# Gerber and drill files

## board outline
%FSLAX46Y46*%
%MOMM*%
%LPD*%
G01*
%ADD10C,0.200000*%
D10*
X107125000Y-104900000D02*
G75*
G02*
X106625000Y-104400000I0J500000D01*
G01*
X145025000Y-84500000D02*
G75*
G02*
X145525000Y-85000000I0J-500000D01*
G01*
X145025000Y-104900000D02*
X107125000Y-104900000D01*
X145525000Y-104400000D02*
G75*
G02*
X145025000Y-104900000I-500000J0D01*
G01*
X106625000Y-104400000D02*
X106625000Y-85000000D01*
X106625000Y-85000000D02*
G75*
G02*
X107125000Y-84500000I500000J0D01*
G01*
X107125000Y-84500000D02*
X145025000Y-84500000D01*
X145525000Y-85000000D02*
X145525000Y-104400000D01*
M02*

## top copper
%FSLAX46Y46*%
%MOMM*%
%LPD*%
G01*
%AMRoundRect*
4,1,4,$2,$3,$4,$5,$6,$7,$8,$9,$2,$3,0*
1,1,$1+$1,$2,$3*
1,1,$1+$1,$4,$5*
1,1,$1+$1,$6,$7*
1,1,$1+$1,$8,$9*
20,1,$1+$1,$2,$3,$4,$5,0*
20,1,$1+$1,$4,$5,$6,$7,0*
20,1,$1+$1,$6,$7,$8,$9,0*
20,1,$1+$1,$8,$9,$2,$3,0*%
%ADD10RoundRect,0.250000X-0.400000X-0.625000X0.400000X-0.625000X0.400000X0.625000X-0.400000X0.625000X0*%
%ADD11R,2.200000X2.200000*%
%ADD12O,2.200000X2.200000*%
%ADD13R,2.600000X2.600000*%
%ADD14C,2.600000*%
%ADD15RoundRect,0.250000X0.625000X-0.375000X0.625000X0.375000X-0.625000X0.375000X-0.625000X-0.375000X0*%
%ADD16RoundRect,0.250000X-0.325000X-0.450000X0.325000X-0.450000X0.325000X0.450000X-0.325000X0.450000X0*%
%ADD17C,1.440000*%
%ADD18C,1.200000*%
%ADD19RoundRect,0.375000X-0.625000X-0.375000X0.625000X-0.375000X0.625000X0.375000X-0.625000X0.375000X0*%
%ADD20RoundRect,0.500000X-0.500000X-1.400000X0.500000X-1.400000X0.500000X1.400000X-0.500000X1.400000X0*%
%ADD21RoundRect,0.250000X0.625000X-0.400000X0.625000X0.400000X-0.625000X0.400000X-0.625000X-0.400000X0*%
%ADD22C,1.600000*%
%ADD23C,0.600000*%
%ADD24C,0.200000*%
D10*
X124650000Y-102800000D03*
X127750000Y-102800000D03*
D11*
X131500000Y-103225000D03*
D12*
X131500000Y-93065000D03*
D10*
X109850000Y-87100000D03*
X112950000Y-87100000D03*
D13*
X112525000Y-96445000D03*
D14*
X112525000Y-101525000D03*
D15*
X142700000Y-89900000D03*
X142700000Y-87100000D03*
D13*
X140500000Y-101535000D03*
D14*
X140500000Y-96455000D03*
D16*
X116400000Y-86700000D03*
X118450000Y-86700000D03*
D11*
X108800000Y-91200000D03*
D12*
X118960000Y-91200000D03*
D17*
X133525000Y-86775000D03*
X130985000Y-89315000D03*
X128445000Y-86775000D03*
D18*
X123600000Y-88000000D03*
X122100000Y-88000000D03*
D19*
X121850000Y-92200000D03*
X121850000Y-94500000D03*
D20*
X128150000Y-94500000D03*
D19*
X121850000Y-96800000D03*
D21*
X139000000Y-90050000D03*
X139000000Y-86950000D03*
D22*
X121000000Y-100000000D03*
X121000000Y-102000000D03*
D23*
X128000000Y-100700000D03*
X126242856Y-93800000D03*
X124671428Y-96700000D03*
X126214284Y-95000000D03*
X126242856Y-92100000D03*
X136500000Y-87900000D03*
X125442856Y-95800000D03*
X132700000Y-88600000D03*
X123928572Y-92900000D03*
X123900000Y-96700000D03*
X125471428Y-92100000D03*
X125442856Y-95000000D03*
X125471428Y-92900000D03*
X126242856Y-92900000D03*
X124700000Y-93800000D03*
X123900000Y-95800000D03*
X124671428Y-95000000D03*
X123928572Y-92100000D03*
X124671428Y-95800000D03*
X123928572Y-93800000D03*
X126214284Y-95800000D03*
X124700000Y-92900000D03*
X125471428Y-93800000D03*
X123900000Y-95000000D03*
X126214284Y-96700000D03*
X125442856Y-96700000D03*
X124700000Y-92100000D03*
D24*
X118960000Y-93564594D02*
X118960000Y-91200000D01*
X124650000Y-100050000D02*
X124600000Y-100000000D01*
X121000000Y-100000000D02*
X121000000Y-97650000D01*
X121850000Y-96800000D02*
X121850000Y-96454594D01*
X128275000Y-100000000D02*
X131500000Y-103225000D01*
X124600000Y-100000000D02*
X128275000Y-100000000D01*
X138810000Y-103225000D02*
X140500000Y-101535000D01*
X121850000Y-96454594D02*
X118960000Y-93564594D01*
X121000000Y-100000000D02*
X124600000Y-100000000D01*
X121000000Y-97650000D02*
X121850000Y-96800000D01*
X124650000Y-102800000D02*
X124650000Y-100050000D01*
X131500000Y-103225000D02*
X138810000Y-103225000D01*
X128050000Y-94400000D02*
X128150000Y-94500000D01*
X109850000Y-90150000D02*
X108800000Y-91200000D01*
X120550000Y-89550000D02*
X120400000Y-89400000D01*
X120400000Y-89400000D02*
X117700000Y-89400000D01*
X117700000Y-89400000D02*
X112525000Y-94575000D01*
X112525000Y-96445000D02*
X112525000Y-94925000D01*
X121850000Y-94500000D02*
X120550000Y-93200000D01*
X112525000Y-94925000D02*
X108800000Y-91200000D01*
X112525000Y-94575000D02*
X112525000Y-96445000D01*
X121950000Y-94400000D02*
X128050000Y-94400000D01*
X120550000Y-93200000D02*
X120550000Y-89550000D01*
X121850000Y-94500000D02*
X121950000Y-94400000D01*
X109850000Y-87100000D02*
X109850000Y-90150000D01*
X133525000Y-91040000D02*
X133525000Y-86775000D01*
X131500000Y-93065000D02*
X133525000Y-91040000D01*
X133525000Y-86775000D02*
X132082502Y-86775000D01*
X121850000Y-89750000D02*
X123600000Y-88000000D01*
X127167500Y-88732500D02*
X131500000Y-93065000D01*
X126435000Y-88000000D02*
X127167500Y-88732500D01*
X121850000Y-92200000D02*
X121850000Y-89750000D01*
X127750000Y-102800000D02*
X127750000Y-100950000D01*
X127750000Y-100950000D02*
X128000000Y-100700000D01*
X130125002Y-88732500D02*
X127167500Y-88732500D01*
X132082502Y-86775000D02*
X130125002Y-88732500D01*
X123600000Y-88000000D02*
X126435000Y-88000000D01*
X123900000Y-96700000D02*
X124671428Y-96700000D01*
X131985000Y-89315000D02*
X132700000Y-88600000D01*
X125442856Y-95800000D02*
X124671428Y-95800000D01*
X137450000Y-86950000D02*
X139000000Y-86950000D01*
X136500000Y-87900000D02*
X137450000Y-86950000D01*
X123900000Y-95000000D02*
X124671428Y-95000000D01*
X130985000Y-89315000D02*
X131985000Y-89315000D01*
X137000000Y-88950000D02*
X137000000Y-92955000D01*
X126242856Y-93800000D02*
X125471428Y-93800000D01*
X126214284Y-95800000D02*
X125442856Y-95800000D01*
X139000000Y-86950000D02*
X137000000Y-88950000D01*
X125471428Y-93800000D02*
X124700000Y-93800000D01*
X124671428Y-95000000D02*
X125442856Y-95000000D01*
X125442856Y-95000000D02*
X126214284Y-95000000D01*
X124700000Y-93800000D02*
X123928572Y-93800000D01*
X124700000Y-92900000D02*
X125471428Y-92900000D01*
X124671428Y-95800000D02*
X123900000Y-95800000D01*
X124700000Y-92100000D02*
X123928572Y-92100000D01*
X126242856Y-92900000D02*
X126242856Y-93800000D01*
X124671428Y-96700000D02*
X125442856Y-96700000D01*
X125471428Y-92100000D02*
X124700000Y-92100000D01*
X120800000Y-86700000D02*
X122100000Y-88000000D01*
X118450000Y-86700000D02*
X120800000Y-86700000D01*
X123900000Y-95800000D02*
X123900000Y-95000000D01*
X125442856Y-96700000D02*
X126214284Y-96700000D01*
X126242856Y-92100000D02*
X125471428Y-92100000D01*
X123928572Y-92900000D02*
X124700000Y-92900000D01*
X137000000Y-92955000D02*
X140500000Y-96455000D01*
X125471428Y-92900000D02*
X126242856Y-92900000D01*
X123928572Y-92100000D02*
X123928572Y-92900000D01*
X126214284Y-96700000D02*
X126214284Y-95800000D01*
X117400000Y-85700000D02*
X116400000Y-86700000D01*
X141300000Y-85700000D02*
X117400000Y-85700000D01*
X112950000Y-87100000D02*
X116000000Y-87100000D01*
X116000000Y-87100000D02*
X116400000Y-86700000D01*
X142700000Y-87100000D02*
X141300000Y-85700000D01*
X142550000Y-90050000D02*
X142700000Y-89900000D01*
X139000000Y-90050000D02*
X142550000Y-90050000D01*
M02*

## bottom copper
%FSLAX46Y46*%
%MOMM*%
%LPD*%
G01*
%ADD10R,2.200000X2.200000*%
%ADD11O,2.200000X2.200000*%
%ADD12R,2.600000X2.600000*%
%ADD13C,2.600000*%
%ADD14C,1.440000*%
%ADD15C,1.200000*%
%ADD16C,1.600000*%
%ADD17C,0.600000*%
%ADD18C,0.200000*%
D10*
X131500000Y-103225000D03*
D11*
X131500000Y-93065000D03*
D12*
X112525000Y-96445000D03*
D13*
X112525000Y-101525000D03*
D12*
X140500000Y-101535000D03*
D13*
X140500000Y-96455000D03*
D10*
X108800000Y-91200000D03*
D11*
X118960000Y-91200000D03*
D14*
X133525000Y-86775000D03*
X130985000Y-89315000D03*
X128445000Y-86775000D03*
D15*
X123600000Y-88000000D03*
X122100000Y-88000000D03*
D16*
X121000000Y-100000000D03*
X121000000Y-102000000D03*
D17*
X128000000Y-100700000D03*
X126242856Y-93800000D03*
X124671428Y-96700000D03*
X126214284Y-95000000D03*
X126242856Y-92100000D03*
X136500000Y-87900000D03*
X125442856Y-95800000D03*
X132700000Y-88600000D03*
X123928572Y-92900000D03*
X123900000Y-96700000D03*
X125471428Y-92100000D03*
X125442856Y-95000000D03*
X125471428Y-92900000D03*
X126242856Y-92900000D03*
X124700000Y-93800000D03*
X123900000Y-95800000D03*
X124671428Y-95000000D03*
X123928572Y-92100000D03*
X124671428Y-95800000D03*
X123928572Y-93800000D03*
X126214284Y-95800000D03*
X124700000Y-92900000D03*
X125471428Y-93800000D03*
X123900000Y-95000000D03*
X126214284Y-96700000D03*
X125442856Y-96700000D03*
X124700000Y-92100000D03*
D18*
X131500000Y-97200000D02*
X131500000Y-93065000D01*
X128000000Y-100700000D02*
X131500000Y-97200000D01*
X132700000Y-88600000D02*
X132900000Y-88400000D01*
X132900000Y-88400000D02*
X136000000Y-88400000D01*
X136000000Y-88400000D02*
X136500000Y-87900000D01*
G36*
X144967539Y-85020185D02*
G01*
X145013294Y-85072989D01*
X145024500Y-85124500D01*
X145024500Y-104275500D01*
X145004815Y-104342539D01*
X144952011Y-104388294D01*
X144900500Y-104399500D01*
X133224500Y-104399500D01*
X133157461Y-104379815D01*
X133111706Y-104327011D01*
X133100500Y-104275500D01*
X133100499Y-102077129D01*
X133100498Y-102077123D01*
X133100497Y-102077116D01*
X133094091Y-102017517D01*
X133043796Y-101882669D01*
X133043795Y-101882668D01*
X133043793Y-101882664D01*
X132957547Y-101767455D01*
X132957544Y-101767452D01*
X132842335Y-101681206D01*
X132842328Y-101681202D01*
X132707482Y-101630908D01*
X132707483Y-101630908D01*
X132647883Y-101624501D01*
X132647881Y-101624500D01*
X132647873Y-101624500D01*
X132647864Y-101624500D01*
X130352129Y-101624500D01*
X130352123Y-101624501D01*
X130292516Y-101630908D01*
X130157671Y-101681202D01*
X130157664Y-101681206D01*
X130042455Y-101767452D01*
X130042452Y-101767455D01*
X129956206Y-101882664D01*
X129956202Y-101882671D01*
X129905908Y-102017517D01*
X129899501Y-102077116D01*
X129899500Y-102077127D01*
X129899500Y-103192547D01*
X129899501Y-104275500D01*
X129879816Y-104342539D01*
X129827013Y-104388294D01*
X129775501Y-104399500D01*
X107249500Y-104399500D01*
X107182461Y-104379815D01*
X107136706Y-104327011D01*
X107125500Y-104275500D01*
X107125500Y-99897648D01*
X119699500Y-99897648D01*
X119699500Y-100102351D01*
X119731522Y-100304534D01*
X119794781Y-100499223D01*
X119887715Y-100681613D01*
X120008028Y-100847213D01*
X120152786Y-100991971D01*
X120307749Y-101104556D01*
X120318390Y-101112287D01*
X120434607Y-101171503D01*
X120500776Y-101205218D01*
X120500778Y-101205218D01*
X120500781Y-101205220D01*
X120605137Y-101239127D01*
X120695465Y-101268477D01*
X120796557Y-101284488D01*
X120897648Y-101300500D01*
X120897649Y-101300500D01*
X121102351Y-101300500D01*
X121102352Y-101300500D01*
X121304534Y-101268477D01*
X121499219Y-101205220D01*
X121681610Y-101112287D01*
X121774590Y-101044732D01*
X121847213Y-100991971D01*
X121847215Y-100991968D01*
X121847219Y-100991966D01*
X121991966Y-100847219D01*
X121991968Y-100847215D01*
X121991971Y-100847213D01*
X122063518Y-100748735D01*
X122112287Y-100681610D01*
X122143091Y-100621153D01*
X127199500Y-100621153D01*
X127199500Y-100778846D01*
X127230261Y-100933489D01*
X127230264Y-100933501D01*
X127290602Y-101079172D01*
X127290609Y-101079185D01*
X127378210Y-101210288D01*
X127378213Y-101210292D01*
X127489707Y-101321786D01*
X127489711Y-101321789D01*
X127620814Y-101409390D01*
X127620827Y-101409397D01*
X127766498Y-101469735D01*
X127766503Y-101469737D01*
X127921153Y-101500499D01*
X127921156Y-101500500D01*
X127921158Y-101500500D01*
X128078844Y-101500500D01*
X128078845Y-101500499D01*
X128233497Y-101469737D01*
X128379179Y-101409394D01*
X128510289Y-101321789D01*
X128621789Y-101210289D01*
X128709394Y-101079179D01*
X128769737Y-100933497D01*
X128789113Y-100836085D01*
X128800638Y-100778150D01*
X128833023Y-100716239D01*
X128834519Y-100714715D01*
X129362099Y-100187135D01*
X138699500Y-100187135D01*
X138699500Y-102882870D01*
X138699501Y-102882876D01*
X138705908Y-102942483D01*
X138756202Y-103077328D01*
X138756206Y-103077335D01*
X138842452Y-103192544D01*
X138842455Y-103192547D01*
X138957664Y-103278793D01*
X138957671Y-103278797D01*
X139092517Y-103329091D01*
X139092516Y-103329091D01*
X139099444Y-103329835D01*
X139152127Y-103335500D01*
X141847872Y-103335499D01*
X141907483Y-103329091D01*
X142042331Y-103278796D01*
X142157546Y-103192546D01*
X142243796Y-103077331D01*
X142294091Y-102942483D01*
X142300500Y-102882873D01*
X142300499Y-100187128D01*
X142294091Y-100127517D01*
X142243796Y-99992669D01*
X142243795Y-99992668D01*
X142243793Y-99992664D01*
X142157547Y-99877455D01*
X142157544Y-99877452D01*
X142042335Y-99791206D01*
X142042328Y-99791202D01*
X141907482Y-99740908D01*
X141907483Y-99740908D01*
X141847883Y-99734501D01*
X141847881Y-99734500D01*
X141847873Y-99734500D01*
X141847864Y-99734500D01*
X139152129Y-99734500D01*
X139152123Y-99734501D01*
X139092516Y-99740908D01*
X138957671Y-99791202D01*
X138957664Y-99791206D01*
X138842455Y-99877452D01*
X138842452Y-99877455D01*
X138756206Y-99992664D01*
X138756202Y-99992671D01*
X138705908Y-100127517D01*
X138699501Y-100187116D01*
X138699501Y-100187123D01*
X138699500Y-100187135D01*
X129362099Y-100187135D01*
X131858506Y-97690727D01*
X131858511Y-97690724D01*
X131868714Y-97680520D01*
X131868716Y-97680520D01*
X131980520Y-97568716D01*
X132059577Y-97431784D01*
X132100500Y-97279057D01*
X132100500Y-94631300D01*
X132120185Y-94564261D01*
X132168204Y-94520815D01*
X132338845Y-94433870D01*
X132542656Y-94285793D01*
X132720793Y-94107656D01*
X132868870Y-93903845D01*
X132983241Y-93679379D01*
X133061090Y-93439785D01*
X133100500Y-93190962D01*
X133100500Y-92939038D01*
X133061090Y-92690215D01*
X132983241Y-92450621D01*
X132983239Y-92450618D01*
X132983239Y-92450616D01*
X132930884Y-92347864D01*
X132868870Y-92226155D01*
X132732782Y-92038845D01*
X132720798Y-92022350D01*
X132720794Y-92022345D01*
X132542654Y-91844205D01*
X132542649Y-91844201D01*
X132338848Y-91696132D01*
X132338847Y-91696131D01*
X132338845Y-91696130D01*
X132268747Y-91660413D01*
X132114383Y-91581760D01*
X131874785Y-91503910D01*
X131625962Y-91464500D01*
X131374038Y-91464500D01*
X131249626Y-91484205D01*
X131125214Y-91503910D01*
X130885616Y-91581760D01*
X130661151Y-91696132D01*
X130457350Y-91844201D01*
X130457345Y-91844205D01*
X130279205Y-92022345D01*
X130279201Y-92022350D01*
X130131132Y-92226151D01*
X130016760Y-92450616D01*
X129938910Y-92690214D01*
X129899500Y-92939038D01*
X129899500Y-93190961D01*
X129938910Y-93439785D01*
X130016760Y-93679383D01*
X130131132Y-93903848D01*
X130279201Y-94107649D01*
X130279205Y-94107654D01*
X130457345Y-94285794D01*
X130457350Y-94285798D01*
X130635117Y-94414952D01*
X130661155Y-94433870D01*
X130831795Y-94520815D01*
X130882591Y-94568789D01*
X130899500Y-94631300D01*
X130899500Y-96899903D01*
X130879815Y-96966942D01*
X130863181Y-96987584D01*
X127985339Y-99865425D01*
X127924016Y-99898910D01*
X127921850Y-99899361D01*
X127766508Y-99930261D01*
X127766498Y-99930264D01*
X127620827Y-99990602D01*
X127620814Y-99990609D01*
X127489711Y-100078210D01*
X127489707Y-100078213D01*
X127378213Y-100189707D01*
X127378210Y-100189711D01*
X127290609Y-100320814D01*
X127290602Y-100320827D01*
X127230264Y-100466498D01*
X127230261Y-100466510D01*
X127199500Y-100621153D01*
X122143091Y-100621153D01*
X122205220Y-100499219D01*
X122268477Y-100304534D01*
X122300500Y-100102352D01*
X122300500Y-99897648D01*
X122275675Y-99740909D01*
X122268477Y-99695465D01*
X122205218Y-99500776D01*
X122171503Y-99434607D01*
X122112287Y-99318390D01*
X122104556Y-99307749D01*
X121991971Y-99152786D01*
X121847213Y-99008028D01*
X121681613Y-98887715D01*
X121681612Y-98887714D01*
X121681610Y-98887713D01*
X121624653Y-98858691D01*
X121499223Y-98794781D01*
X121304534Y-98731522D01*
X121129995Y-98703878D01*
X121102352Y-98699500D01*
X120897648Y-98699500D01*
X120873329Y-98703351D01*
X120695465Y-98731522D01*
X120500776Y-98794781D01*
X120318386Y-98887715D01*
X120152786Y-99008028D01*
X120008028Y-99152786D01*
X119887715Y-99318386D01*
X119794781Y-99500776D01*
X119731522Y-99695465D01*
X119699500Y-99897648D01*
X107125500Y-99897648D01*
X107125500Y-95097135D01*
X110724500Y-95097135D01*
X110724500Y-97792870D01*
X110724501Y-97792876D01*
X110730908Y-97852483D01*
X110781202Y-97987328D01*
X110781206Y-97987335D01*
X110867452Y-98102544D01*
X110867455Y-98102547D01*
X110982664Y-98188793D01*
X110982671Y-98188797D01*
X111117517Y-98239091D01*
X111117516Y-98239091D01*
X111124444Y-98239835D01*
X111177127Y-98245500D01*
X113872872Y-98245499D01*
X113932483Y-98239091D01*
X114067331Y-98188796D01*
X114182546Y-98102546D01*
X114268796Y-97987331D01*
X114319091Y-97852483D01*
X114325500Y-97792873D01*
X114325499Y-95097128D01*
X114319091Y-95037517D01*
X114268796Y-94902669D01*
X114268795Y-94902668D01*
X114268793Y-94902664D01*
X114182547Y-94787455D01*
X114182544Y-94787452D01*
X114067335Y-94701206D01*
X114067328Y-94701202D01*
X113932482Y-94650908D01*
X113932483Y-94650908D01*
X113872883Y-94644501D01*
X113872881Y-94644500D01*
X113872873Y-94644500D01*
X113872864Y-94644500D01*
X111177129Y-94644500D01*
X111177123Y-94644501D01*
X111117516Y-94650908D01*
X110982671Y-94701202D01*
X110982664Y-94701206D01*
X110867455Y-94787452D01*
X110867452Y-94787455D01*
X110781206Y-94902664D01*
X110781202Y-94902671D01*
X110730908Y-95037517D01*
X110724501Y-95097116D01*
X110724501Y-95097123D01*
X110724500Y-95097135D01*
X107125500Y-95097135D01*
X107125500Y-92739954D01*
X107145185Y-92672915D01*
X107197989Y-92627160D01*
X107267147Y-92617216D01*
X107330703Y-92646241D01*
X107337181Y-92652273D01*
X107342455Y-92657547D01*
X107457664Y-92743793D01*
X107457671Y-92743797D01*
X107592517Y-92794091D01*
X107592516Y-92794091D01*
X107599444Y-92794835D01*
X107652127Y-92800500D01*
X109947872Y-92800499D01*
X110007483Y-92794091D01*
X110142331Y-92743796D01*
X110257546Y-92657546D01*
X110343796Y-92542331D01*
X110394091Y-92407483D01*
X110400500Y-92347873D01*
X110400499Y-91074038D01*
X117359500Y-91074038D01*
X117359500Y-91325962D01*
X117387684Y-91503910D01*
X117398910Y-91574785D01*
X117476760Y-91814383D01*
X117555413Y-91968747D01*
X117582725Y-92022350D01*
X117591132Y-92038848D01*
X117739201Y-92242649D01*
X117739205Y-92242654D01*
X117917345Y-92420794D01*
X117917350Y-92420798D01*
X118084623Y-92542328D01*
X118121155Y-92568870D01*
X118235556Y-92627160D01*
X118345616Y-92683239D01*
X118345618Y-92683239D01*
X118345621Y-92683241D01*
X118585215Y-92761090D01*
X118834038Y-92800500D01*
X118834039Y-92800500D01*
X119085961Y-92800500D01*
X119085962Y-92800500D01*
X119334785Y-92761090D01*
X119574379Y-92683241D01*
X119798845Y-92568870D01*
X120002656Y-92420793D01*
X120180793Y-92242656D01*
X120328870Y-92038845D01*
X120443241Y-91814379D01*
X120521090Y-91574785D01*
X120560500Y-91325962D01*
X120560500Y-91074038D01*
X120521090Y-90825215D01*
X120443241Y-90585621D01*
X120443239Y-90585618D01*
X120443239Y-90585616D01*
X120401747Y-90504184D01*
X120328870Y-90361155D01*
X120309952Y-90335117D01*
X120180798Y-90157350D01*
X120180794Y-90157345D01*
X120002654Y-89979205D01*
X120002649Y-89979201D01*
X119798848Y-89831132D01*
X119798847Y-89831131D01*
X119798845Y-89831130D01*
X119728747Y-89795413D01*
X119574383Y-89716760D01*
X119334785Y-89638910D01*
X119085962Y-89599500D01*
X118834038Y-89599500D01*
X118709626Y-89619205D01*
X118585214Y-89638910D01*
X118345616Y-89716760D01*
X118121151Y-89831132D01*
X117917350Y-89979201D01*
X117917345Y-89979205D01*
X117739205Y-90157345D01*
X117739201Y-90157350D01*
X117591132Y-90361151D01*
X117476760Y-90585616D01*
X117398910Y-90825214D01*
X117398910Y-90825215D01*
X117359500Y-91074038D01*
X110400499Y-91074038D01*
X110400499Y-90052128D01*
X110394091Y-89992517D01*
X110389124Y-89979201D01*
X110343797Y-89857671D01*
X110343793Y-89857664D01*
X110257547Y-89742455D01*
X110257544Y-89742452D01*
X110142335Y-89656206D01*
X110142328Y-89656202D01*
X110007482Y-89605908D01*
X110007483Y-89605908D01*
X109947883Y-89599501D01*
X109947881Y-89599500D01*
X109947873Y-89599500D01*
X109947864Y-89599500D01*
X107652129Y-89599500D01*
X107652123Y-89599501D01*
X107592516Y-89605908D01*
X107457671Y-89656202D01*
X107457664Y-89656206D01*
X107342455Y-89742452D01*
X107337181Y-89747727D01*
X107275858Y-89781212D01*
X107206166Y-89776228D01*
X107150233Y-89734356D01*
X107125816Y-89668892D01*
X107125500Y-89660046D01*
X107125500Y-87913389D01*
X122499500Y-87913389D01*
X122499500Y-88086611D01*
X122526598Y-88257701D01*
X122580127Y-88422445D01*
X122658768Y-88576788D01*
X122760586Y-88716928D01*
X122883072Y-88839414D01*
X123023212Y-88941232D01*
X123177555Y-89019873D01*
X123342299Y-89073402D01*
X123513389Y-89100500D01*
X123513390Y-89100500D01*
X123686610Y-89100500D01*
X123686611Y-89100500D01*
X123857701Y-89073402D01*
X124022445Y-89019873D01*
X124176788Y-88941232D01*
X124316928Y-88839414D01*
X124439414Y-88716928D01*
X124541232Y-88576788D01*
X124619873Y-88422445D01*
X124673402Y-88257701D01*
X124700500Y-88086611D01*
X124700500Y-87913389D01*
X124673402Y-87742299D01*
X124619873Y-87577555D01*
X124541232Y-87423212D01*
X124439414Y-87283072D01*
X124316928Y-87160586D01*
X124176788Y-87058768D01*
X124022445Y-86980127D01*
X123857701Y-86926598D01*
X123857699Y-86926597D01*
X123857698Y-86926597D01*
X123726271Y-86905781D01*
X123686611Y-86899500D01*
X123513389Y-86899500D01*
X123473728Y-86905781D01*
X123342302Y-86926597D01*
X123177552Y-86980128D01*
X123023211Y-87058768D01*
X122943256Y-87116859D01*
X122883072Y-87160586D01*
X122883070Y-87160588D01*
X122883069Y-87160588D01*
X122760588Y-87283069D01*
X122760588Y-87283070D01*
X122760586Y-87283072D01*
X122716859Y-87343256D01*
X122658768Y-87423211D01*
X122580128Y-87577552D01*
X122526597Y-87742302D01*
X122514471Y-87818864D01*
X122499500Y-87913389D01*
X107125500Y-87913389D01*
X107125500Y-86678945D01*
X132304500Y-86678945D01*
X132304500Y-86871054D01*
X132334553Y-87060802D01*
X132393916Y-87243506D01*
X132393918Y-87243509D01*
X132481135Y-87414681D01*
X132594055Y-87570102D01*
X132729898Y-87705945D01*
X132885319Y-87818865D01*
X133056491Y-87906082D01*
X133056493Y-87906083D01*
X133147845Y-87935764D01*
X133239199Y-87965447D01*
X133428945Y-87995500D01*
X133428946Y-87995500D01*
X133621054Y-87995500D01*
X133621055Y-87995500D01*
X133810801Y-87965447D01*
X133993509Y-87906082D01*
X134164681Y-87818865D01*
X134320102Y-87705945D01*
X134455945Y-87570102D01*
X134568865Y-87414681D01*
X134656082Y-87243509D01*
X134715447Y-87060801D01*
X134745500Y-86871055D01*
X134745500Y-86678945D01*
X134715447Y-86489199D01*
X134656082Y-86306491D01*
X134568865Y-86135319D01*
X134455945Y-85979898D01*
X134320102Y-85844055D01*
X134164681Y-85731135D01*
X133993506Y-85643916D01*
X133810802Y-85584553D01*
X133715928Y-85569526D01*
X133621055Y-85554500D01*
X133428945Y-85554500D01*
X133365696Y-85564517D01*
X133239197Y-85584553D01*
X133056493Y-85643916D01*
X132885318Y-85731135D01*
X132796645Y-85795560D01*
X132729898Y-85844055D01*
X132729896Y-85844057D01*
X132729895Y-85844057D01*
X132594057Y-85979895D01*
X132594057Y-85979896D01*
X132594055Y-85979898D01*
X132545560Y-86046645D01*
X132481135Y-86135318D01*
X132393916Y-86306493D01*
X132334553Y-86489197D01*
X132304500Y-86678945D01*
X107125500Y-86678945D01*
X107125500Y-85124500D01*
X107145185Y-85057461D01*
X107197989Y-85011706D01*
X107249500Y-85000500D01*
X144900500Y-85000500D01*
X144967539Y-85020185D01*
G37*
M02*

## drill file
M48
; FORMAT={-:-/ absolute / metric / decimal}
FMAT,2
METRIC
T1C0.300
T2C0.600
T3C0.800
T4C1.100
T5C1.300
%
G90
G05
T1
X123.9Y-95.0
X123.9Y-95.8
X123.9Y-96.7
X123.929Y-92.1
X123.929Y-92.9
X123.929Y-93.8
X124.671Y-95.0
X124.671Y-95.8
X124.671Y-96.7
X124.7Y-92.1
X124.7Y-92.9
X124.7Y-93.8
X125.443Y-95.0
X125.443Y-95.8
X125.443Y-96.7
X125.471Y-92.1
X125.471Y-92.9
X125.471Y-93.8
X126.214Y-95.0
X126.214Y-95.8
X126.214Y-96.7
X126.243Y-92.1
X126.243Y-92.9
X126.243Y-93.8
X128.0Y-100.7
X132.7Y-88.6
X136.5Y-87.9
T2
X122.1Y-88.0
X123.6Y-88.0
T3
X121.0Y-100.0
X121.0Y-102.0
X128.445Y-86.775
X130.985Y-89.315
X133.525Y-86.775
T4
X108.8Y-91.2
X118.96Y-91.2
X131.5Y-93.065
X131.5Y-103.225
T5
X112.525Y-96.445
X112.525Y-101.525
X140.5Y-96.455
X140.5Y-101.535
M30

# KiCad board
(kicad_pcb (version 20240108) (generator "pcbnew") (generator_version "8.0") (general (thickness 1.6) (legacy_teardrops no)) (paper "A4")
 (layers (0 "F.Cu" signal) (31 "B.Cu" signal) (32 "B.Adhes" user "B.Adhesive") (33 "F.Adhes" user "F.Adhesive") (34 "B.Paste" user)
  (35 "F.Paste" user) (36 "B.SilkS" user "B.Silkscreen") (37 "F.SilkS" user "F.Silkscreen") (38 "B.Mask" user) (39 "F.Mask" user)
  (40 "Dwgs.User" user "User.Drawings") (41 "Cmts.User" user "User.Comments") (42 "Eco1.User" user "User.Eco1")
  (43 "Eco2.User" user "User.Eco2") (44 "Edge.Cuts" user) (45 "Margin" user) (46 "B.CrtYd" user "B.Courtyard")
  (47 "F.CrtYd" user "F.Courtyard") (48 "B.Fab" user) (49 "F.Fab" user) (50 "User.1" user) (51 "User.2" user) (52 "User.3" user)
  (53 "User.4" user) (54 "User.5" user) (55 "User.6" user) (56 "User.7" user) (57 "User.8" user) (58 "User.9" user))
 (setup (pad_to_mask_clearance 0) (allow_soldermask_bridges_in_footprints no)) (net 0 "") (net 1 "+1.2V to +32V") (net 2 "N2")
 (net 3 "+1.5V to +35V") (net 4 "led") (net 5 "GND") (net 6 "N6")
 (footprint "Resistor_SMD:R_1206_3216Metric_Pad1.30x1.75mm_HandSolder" (layer "F.Cu") (at 126.2 102.8)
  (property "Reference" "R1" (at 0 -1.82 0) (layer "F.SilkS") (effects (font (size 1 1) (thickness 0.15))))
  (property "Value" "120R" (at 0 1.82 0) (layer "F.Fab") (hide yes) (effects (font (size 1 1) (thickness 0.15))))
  (pad "1" smd roundrect (at -1.55 0) (size 1.3 1.75) (layers "F.Cu" "F.Paste" "F.Mask") (roundrect_rratio 0.192308) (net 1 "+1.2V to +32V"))
  (pad "2" smd roundrect (at 1.55 0) (size 1.3 1.75) (layers "F.Cu" "F.Paste" "F.Mask") (roundrect_rratio 0.192308) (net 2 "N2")))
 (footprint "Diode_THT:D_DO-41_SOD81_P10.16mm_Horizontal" (layer "F.Cu") (at 131.5 103.225 90)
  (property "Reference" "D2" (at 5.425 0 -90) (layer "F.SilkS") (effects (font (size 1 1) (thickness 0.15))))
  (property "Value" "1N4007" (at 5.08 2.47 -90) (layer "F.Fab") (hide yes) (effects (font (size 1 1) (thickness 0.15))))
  (pad "1" thru_hole rect (at 0 0 90) (size 2.2 2.2) (drill 1.1) (layers "*.Cu" "*.Mask") (remove_unused_layers no) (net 1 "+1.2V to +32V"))
  (pad "2" thru_hole oval (at 10.16 0 90) (size 2.2 2.2) (drill 1.1) (layers "*.Cu" "*.Mask") (remove_unused_layers no) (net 2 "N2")))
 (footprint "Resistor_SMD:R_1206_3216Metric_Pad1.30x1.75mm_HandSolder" (layer "F.Cu") (at 111.4 87.1)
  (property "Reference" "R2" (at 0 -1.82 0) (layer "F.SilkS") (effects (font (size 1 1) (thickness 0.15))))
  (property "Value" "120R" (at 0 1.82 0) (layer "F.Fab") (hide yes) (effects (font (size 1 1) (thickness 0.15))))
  (pad "1" smd roundrect (at -1.55 0) (size 1.3 1.75) (layers "F.Cu" "F.Paste" "F.Mask") (roundrect_rratio 0.192308) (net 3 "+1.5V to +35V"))
  (pad "2" smd roundrect (at 1.55 0) (size 1.3 1.75) (layers "F.Cu" "F.Paste" "F.Mask") (roundrect_rratio 0.192308) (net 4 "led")))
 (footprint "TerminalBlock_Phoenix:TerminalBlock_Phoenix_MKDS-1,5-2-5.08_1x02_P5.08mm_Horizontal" (layer "F.Cu") (at 112.525 96.445 -90)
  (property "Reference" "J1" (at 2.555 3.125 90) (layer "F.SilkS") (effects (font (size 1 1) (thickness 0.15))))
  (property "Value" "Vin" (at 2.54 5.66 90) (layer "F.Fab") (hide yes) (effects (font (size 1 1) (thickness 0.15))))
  (pad "1" thru_hole rect (at 0 0 270) (size 2.6 2.6) (drill 1.3) (layers "*.Cu" "*.Mask") (remove_unused_layers no) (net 3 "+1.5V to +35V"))
  (pad "2" thru_hole circle (at 5.08 0 270) (size 2.6 2.6) (drill 1.3) (layers "*.Cu" "*.Mask") (remove_unused_layers no) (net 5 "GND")))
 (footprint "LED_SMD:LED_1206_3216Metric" (layer "F.Cu") (at 142.7 88.5 90)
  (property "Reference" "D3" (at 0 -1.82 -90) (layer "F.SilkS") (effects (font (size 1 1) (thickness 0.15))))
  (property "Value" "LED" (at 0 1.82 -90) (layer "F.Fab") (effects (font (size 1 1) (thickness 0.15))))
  (pad "1" smd roundrect (at -1.4 0 90) (size 1.25 1.75) (layers "F.Cu" "F.Paste" "F.Mask") (roundrect_rratio 0.2) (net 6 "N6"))
  (pad "2" smd roundrect (at 1.4 0 90) (size 1.25 1.75) (layers "F.Cu" "F.Paste" "F.Mask") (roundrect_rratio 0.2) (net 4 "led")))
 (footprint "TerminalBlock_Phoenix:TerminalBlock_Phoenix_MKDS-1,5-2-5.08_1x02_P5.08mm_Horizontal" (layer "F.Cu") (at 140.5 101.535 90)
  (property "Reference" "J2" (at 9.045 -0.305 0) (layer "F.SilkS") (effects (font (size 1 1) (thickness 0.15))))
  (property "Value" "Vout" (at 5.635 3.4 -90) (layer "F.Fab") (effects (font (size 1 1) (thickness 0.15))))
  (pad "1" thru_hole rect (at 0 0 90) (size 2.6 2.6) (drill 1.3) (layers "*.Cu" "*.Mask") (remove_unused_layers no) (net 1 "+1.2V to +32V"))
  (pad "2" thru_hole circle (at 5.08 0 90) (size 2.6 2.6) (drill 1.3) (layers "*.Cu" "*.Mask") (remove_unused_layers no) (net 5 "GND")))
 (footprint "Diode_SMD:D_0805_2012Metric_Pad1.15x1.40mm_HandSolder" (layer "F.Cu") (at 117.425 86.7)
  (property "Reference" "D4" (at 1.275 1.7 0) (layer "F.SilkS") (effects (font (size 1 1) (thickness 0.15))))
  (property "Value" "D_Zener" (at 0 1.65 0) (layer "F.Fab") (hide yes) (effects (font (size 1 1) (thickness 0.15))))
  (pad "1" smd roundrect (at -1.025 0) (size 1.15 1.4) (layers "F.Cu" "F.Paste" "F.Mask") (roundrect_rratio 0.217391) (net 4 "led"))
  (pad "2" smd roundrect (at 1.025 0) (size 1.15 1.4) (layers "F.Cu" "F.Paste" "F.Mask") (roundrect_rratio 0.217391) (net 5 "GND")))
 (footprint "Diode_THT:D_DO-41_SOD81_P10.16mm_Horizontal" (layer "F.Cu") (at 108.8 91.2)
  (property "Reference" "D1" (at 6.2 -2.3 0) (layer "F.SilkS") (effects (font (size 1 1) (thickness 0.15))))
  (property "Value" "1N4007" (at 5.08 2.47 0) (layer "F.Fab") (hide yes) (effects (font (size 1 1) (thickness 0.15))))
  (pad "1" thru_hole rect (at 0 0) (size 2.2 2.2) (drill 1.1) (layers "*.Cu" "*.Mask") (remove_unused_layers no) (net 3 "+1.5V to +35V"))
  (pad "2" thru_hole oval (at 10.16 0) (size 2.2 2.2) (drill 1.1) (layers "*.Cu" "*.Mask") (remove_unused_layers no) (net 1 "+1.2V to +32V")))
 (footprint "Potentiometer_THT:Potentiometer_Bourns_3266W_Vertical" (layer "F.Cu") (at 133.525 86.775)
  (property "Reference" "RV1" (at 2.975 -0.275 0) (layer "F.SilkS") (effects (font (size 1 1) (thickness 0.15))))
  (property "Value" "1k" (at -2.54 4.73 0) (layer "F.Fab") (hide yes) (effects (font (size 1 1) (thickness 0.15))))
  (pad "1" thru_hole circle (at 0 0) (size 1.44 1.44) (drill 0.8) (layers "*.Cu" "*.Mask") (remove_unused_layers no) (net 2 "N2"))
  (pad "2" thru_hole circle (at -2.54 2.54) (size 1.44 1.44) (drill 0.8) (layers "*.Cu" "*.Mask") (remove_unused_layers no) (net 5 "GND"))
  (pad "3" thru_hole circle (at -5.08 0) (size 1.44 1.44) (drill 0.8) (layers "*.Cu" "*.Mask") (remove_unused_layers no) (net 5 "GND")))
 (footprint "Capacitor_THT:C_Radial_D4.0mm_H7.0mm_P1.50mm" (layer "F.Cu") (at 123.6 88 180)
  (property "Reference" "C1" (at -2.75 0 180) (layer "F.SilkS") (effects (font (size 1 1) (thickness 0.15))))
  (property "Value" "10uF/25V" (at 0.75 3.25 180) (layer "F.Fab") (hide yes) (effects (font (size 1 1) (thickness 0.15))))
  (pad "1" thru_hole circle (at 0 0 180) (size 1.2 1.2) (drill 0.6) (layers "*.Cu" "*.Mask") (remove_unused_layers no) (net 2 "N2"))
  (pad "2" thru_hole circle (at 1.5 0 180) (size 1.2 1.2) (drill 0.6) (layers "*.Cu" "*.Mask") (remove_unused_layers no) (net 5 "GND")))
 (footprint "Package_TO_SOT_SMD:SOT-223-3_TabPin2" (layer "F.Cu") (at 125 94.5)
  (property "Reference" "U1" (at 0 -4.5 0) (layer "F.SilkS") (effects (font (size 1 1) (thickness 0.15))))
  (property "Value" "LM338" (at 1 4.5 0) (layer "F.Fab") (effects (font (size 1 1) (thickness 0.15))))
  (pad "1" smd roundrect (at -3.15 -2.3) (size 2 1.5) (layers "F.Cu" "F.Paste" "F.Mask") (roundrect_rratio 0.25) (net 2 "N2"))
  (pad "2" smd roundrect (at -3.15 0) (size 2 1.5) (layers "F.Cu" "F.Paste" "F.Mask") (roundrect_rratio 0.25) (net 3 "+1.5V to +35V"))
  (pad "2" smd roundrect (at 3.15 0) (size 2 3.8) (layers "F.Cu" "F.Paste" "F.Mask") (roundrect_rratio 0.25) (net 3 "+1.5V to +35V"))
  (pad "3" smd roundrect (at -3.15 2.3) (size 2 1.5) (layers "F.Cu" "F.Paste" "F.Mask") (roundrect_rratio 0.25) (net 1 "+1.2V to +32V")))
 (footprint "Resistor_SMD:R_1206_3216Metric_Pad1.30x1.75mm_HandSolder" (layer "F.Cu") (at 139 88.5 90)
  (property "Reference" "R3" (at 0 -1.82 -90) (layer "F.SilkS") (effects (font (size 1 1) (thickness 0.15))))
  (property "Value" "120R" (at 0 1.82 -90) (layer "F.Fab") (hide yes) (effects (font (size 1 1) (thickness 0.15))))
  (pad "1" smd roundrect (at -1.55 0 90) (size 1.3 1.75) (layers "F.Cu" "F.Paste" "F.Mask") (roundrect_rratio 0.192308) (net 6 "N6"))
  (pad "2" smd roundrect (at 1.55 0 90) (size 1.3 1.75) (layers "F.Cu" "F.Paste" "F.Mask") (roundrect_rratio 0.192308) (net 5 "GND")))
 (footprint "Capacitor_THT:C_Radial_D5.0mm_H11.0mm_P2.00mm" (layer "F.Cu") (at 121 100 -90)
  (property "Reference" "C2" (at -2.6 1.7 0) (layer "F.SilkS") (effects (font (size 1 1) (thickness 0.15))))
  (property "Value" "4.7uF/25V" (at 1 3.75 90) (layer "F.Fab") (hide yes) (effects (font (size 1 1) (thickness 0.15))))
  (pad "1" thru_hole circle (at 0 0 270) (size 1.6 1.6) (drill 0.8) (layers "*.Cu" "*.Mask") (remove_unused_layers no)
   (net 1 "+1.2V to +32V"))
  (pad "2" thru_hole circle (at 2 0 270) (size 1.6 1.6) (drill 0.8) (layers "*.Cu" "*.Mask") (remove_unused_layers no) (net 5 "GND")))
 (gr_arc (start 107.125 104.9) (mid 106.771447 104.753553) (end 106.625 104.4) (stroke (width 0.2) (type default)) (layer "Edge.Cuts"))
 (gr_arc (start 145.025 84.5) (mid 145.378553 84.646447) (end 145.525 85) (stroke (width 0.2) (type default)) (layer "Edge.Cuts"))
 (gr_line (start 145.025 104.9) (end 107.125 104.9) (stroke (width 0.2) (type default)) (layer "Edge.Cuts"))
 (gr_arc (start 145.525 104.4) (mid 145.378553 104.753553) (end 145.025 104.9) (stroke (width 0.2) (type default)) (layer "Edge.Cuts"))
 (gr_line (start 106.625 104.4) (end 106.625 85) (stroke (width 0.2) (type default)) (layer "Edge.Cuts"))
 (gr_arc (start 106.625 85) (mid 106.771447 84.646447) (end 107.125 84.5) (stroke (width 0.2) (type default)) (layer "Edge.Cuts"))
 (gr_line (start 107.125 84.5) (end 145.025 84.5) (stroke (width 0.2) (type default)) (layer "Edge.Cuts"))
 (gr_line (start 145.525 85) (end 145.525 104.4) (stroke (width 0.2) (type default)) (layer "Edge.Cuts"))
 (segment (start 118.96 93.564594) (end 118.96 91.2) (width 0.2) (layer "F.Cu") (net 1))
 (segment (start 124.65 100.05) (end 124.6 100) (width 0.2) (layer "F.Cu") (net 1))
 (segment (start 121 100) (end 121 97.65) (width 0.2) (layer "F.Cu") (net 1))
 (segment (start 121.85 96.8) (end 121.85 96.454594) (width 0.2) (layer "F.Cu") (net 1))
 (segment (start 128.275 100) (end 131.5 103.225) (width 0.2) (layer "F.Cu") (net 1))
 (segment (start 124.6 100) (end 128.275 100) (width 0.2) (layer "F.Cu") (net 1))
 (segment (start 138.81 103.225) (end 140.5 101.535) (width 0.2) (layer "F.Cu") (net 1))
 (segment (start 121.85 96.454594) (end 118.96 93.564594) (width 0.2) (layer "F.Cu") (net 1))
 (segment (start 121 100) (end 124.6 100) (width 0.2) (layer "F.Cu") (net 1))
 (segment (start 121 97.65) (end 121.85 96.8) (width 0.2) (layer "F.Cu") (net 1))
 (segment (start 124.65 102.8) (end 124.65 100.05) (width 0.2) (layer "F.Cu") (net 1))
 (segment (start 131.5 103.225) (end 138.81 103.225) (width 0.2) (layer "F.Cu") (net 1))
 (segment (start 128.05 94.4) (end 128.15 94.5) (width 0.2) (layer "F.Cu") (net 3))
 (segment (start 109.85 90.15) (end 108.8 91.2) (width 0.2) (layer "F.Cu") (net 3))
 (segment (start 120.55 89.55) (end 120.4 89.4) (width 0.2) (layer "F.Cu") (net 3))
 (segment (start 120.4 89.4) (end 117.7 89.4) (width 0.2) (layer "F.Cu") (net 3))
 (segment (start 117.7 89.4) (end 112.525 94.575) (width 0.2) (layer "F.Cu") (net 3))
 (segment (start 112.525 96.445) (end 112.525 94.925) (width 0.2) (layer "F.Cu") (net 3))
 (segment (start 121.85 94.5) (end 120.55 93.2) (width 0.2) (layer "F.Cu") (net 3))
 (segment (start 112.525 94.925) (end 108.8 91.2) (width 0.2) (layer "F.Cu") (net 3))
 (segment (start 112.525 94.575) (end 112.525 96.445) (width 0.2) (layer "F.Cu") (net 3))
 (segment (start 121.95 94.4) (end 128.05 94.4) (width 0.2) (layer "F.Cu") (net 3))
 (segment (start 120.55 93.2) (end 120.55 89.55) (width 0.2) (layer "F.Cu") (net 3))
 (segment (start 121.85 94.5) (end 121.95 94.4) (width 0.2) (layer "F.Cu") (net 3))
 (segment (start 109.85 87.1) (end 109.85 90.15) (width 0.2) (layer "F.Cu") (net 3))
 (segment (start 133.525 91.04) (end 133.525 86.775) (width 0.2) (layer "F.Cu") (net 2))
 (segment (start 131.5 93.065) (end 133.525 91.04) (width 0.2) (layer "F.Cu") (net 2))
 (segment (start 133.525 86.775) (end 132.082502 86.775) (width 0.2) (layer "F.Cu") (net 2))
 (segment (start 121.85 89.75) (end 123.6 88) (width 0.2) (layer "F.Cu") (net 2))
 (segment (start 127.1675 88.7325) (end 131.5 93.065) (width 0.2) (layer "F.Cu") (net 2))
 (segment (start 126.435 88) (end 127.1675 88.7325) (width 0.2) (layer "F.Cu") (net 2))
 (segment (start 121.85 92.2) (end 121.85 89.75) (width 0.2) (layer "F.Cu") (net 2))
 (segment (start 127.75 102.8) (end 127.75 100.95) (width 0.2) (layer "F.Cu") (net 2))
 (segment (start 127.75 100.95) (end 128 100.7) (width 0.2) (layer "F.Cu") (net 2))
 (segment (start 130.125002 88.7325) (end 127.1675 88.7325) (width 0.2) (layer "F.Cu") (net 2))
 (segment (start 132.082502 86.775) (end 130.125002 88.7325) (width 0.2) (layer "F.Cu") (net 2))
 (segment (start 123.6 88) (end 126.435 88) (width 0.2) (layer "F.Cu") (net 2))
 (via (at 128 100.7) (size 0.6) (drill 0.3) (layers "F.Cu" "B.Cu") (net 2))
 (segment (start 131.5 97.2) (end 131.5 93.065) (width 0.2) (layer "B.Cu") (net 2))
 (segment (start 128 100.7) (end 131.5 97.2) (width 0.2) (layer "B.Cu") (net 2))
 (segment (start 123.9 96.7) (end 124.671428 96.7) (width 0.2) (layer "F.Cu") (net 5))
 (segment (start 131.985 89.315) (end 132.7 88.6) (width 0.2) (layer "F.Cu") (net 5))
 (segment (start 125.442856 95.8) (end 124.671428 95.8) (width 0.2) (layer "F.Cu") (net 5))
 (segment (start 137.45 86.95) (end 139 86.95) (width 0.2) (layer "F.Cu") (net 5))
 (segment (start 136.5 87.9) (end 137.45 86.95) (width 0.2) (layer "F.Cu") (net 5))
 (segment (start 123.9 95) (end 124.671428 95) (width 0.2) (layer "F.Cu") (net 5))
 (segment (start 130.985 89.315) (end 131.985 89.315) (width 0.2) (layer "F.Cu") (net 5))
 (segment (start 137 88.95) (end 137 92.955) (width 0.2) (layer "F.Cu") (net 5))
 (segment (start 126.242856 93.8) (end 125.471428 93.8) (width 0.2) (layer "F.Cu") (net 5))
 (segment (start 126.214284 95.8) (end 125.442856 95.8) (width 0.2) (layer "F.Cu") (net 5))
 (segment (start 139 86.95) (end 137 88.95) (width 0.2) (layer "F.Cu") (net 5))
 (segment (start 125.471428 93.8) (end 124.7 93.8) (width 0.2) (layer "F.Cu") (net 5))
 (segment (start 124.671428 95) (end 125.442856 95) (width 0.2) (layer "F.Cu") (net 5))
 (segment (start 125.442856 95) (end 126.214284 95) (width 0.2) (layer "F.Cu") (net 5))
 (segment (start 124.7 93.8) (end 123.928572 93.8) (width 0.2) (layer "F.Cu") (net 5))
 (segment (start 124.7 92.9) (end 125.471428 92.9) (width 0.2) (layer "F.Cu") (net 5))
 (segment (start 124.671428 95.8) (end 123.9 95.8) (width 0.2) (layer "F.Cu") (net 5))
 (segment (start 124.7 92.1) (end 123.928572 92.1) (width 0.2) (layer "F.Cu") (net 5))
 (segment (start 126.242856 92.9) (end 126.242856 93.8) (width 0.2) (layer "F.Cu") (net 5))
 (segment (start 124.671428 96.7) (end 125.442856 96.7) (width 0.2) (layer "F.Cu") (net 5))
 (segment (start 125.471428 92.1) (end 124.7 92.1) (width 0.2) (layer "F.Cu") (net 5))
 (segment (start 120.8 86.7) (end 122.1 88) (width 0.2) (layer "F.Cu") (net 5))
 (segment (start 118.45 86.7) (end 120.8 86.7) (width 0.2) (layer "F.Cu") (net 5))
 (segment (start 123.9 95.8) (end 123.9 95) (width 0.2) (layer "F.Cu") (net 5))
 (segment (start 125.442856 96.7) (end 126.214284 96.7) (width 0.2) (layer "F.Cu") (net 5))
 (segment (start 126.242856 92.1) (end 125.471428 92.1) (width 0.2) (layer "F.Cu") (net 5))
 (segment (start 123.928572 92.9) (end 124.7 92.9) (width 0.2) (layer "F.Cu") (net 5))
 (segment (start 137 92.955) (end 140.5 96.455) (width 0.2) (layer "F.Cu") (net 5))
 (segment (start 125.471428 92.9) (end 126.242856 92.9) (width 0.2) (layer "F.Cu") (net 5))
 (segment (start 123.928572 92.1) (end 123.928572 92.9) (width 0.2) (layer "F.Cu") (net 5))
 (segment (start 126.214284 96.7) (end 126.214284 95.8) (width 0.2) (layer "F.Cu") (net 5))
 (via (at 126.242856 93.8) (size 0.6) (drill 0.3) (layers "F.Cu" "B.Cu") (free yes) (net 5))
 (via (at 124.671428 96.7) (size 0.6) (drill 0.3) (layers "F.Cu" "B.Cu") (free yes) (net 5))
 (via (at 126.214284 95) (size 0.6) (drill 0.3) (layers "F.Cu" "B.Cu") (free yes) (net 5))
 (via (at 126.242856 92.1) (size 0.6) (drill 0.3) (layers "F.Cu" "B.Cu") (free yes) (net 5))
 (via (at 136.5 87.9) (size 0.6) (drill 0.3) (layers "F.Cu" "B.Cu") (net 5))
 (via (at 125.442856 95.8) (size 0.6) (drill 0.3) (layers "F.Cu" "B.Cu") (free yes) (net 5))
 (via (at 132.7 88.6) (size 0.6) (drill 0.3) (layers "F.Cu" "B.Cu") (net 5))
 (via (at 123.928572 92.9) (size 0.6) (drill 0.3) (layers "F.Cu" "B.Cu") (free yes) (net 5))
 (via (at 123.9 96.7) (size 0.6) (drill 0.3) (layers "F.Cu" "B.Cu") (free yes) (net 5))
 (via (at 125.471428 92.1) (size 0.6) (drill 0.3) (layers "F.Cu" "B.Cu") (free yes) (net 5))
 (via (at 125.442856 95) (size 0.6) (drill 0.3) (layers "F.Cu" "B.Cu") (free yes) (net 5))
 (via (at 125.471428 92.9) (size 0.6) (drill 0.3) (layers "F.Cu" "B.Cu") (free yes) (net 5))
 (via (at 126.242856 92.9) (size 0.6) (drill 0.3) (layers "F.Cu" "B.Cu") (free yes) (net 5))
 (via (at 124.7 93.8) (size 0.6) (drill 0.3) (layers "F.Cu" "B.Cu") (free yes) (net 5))
 (via (at 123.9 95.8) (size 0.6) (drill 0.3) (layers "F.Cu" "B.Cu") (free yes) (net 5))
 (via (at 124.671428 95) (size 0.6) (drill 0.3) (layers "F.Cu" "B.Cu") (free yes) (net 5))
 (via (at 123.928572 92.1) (size 0.6) (drill 0.3) (layers "F.Cu" "B.Cu") (free yes) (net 5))
 (via (at 124.671428 95.8) (size 0.6) (drill 0.3) (layers "F.Cu" "B.Cu") (free yes) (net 5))
 (via (at 123.928572 93.8) (size 0.6) (drill 0.3) (layers "F.Cu" "B.Cu") (free yes) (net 5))
 (via (at 126.214284 95.8) (size 0.6) (drill 0.3) (layers "F.Cu" "B.Cu") (free yes) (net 5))
 (via (at 124.7 92.9) (size 0.6) (drill 0.3) (layers "F.Cu" "B.Cu") (free yes) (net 5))
 (via (at 125.471428 93.8) (size 0.6) (drill 0.3) (layers "F.Cu" "B.Cu") (free yes) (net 5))
 (via (at 123.9 95) (size 0.6) (drill 0.3) (layers "F.Cu" "B.Cu") (free yes) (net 5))
 (via (at 126.214284 96.7) (size 0.6) (drill 0.3) (layers "F.Cu" "B.Cu") (free yes) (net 5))
 (via (at 125.442856 96.7) (size 0.6) (drill 0.3) (layers "F.Cu" "B.Cu") (free yes) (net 5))
 (via (at 124.7 92.1) (size 0.6) (drill 0.3) (layers "F.Cu" "B.Cu") (free yes) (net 5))
 (segment (start 132.7 88.6) (end 132.9 88.4) (width 0.2) (layer "B.Cu") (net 5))
 (segment (start 132.9 88.4) (end 136 88.4) (width 0.2) (layer "B.Cu") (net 5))
 (segment (start 136 88.4) (end 136.5 87.9) (width 0.2) (layer "B.Cu") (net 5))
 (segment (start 117.4 85.7) (end 116.4 86.7) (width 0.2) (layer "F.Cu") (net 4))
 (segment (start 141.3 85.7) (end 117.4 85.7) (width 0.2) (layer "F.Cu") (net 4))
 (segment (start 112.95 87.1) (end 116 87.1) (width 0.2) (layer "F.Cu") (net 4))
 (segment (start 116 87.1) (end 116.4 86.7) (width 0.2) (layer "F.Cu") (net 4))
 (segment (start 142.7 87.1) (end 141.3 85.7) (width 0.2) (layer "F.Cu") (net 4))
 (segment (start 142.55 90.05) (end 142.7 89.9) (width 0.2) (layer "F.Cu") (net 6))
 (segment (start 139 90.05) (end 142.55 90.05) (width 0.2) (layer "F.Cu") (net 6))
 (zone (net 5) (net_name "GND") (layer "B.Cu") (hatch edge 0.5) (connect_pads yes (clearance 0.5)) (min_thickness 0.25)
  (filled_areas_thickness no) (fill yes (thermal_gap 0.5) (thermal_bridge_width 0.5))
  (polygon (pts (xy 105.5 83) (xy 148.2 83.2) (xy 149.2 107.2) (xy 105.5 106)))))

